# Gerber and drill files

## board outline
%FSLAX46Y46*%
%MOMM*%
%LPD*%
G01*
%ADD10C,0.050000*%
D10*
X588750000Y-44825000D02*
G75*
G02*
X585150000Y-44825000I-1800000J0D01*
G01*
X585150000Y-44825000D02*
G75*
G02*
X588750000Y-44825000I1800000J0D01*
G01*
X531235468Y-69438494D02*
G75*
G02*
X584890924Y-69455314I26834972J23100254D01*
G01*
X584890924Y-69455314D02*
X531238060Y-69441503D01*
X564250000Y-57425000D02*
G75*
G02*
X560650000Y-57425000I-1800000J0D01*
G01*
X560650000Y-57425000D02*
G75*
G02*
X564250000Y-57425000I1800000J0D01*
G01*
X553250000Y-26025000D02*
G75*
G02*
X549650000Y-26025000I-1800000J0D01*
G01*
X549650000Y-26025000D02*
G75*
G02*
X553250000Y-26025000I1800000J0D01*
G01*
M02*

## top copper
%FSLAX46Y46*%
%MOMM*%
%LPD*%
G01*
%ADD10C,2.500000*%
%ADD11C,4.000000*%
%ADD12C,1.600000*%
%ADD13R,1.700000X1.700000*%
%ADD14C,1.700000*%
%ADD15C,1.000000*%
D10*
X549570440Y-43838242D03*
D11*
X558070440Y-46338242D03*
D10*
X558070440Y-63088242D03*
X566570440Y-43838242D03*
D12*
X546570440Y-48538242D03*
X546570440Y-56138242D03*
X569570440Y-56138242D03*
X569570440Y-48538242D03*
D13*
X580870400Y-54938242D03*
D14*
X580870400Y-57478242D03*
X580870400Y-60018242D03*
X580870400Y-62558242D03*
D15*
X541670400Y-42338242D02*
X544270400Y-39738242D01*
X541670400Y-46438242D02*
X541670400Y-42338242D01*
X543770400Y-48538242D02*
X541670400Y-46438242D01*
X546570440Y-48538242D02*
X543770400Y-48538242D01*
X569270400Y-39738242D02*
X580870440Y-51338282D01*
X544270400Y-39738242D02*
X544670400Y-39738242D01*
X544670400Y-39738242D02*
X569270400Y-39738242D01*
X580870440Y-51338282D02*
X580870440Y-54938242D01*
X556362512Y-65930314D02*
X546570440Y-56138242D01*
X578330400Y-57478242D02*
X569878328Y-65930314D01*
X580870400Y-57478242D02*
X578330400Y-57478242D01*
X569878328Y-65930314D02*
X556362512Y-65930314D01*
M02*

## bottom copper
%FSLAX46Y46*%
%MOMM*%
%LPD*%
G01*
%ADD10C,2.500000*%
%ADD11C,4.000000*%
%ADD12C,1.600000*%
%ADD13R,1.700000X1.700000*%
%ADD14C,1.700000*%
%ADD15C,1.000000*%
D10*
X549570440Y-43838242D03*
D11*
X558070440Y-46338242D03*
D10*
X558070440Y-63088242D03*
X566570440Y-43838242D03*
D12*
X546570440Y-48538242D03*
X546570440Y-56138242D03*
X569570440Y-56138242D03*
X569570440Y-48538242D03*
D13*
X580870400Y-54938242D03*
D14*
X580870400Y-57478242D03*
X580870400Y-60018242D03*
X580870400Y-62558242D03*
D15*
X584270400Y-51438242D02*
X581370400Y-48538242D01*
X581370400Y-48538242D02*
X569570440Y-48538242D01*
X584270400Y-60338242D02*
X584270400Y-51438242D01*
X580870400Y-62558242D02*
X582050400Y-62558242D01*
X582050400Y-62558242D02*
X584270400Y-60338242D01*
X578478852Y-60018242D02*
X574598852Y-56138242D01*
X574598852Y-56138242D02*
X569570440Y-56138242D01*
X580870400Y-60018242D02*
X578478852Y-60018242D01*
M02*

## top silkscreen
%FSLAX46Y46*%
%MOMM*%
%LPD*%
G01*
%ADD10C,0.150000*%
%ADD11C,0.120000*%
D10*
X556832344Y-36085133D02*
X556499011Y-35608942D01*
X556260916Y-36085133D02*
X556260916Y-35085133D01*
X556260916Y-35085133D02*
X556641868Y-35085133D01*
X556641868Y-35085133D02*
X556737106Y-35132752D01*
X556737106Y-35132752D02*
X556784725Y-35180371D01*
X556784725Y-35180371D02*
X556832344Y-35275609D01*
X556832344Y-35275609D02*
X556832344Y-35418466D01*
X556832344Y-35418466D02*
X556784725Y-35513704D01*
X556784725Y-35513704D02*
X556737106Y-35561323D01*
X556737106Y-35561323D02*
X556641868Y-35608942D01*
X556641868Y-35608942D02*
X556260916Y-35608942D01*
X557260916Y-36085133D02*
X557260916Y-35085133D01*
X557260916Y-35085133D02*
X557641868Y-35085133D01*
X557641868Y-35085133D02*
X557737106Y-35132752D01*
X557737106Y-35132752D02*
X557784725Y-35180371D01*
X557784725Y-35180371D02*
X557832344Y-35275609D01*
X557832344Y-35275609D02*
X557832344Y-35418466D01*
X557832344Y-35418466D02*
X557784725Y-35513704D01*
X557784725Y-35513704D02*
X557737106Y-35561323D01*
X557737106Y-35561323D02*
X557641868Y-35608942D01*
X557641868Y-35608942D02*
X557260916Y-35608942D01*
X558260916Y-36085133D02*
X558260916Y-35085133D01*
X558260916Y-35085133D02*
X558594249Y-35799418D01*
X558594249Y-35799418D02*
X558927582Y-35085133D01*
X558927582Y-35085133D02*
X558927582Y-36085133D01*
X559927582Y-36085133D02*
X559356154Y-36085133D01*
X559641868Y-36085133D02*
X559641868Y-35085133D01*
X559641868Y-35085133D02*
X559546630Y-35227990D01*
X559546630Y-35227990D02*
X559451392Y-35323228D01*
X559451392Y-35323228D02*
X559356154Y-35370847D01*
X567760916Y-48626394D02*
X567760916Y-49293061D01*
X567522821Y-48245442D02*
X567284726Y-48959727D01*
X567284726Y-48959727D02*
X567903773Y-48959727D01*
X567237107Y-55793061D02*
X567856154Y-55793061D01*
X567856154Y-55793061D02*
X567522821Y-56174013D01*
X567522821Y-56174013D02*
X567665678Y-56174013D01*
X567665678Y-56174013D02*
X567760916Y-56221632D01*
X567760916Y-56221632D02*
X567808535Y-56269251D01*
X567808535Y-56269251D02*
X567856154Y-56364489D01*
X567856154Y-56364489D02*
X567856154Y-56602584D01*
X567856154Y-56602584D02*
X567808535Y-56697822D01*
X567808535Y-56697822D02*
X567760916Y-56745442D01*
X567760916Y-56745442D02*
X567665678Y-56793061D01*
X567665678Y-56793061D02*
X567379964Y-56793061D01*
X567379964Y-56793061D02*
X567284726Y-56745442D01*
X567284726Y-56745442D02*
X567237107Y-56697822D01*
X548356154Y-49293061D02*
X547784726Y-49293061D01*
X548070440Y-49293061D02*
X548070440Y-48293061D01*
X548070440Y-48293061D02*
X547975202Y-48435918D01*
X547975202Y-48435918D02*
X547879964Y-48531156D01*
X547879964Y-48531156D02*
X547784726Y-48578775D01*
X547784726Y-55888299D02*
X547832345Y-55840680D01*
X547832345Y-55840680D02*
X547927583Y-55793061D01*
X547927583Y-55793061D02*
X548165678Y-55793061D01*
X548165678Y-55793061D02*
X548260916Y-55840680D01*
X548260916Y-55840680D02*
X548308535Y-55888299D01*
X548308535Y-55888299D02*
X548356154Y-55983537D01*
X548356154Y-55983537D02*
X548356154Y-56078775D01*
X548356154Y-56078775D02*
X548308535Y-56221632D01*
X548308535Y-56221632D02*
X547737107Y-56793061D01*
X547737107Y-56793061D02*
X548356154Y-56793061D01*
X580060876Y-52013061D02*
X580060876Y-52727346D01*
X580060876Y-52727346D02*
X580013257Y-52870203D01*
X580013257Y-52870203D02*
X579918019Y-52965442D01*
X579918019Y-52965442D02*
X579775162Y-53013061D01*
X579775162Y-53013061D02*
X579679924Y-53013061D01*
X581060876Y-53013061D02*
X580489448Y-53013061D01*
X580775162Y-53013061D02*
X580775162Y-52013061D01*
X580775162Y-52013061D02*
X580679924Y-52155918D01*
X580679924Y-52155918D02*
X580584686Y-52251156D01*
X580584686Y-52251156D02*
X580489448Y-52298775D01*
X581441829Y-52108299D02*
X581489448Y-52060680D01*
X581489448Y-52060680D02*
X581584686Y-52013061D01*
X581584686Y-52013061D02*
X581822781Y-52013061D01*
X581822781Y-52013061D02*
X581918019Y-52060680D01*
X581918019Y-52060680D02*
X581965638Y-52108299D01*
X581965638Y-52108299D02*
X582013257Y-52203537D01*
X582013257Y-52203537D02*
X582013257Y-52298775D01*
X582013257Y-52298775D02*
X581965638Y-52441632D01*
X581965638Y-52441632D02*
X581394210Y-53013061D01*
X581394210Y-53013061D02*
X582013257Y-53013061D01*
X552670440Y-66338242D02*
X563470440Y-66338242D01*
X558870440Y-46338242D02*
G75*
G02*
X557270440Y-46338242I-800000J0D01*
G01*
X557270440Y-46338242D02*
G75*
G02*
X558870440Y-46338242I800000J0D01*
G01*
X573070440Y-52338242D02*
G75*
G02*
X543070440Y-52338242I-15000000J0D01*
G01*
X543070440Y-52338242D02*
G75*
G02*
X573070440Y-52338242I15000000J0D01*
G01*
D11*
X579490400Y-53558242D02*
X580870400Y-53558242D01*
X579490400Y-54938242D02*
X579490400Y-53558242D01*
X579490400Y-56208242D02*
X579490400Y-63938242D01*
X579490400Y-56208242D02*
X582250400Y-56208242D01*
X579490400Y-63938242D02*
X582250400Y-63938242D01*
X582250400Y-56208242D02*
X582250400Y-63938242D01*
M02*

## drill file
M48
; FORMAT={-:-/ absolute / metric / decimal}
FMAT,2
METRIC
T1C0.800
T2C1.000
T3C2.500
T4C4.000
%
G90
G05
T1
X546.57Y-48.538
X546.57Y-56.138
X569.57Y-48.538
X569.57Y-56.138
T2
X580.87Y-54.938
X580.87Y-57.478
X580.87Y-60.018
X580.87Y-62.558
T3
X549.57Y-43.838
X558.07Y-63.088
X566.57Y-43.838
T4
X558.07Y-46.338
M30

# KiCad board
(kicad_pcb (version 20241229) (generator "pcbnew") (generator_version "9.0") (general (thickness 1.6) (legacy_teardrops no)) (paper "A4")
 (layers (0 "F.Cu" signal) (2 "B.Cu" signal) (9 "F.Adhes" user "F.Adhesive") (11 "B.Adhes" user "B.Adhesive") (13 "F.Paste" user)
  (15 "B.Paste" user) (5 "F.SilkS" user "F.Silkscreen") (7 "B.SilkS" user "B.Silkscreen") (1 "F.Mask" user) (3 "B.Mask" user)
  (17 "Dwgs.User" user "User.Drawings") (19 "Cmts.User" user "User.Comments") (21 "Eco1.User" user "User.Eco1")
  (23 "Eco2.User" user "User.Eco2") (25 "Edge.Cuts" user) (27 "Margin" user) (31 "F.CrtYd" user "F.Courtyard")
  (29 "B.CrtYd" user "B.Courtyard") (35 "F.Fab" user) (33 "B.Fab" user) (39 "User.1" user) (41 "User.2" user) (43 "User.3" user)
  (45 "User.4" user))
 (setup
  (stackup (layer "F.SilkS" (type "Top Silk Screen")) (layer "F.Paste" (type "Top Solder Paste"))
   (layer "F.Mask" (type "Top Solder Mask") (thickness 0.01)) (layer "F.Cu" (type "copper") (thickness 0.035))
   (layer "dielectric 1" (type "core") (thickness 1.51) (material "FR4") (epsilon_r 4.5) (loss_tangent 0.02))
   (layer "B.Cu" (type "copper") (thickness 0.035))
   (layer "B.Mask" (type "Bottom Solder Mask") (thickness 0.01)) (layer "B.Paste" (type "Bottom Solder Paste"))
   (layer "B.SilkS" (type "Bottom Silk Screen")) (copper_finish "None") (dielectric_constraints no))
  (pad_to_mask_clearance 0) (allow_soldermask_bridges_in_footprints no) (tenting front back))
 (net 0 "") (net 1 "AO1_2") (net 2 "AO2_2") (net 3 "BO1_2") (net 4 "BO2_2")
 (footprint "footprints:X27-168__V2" (layer "F.Cu") (at 558.07044 52.338242)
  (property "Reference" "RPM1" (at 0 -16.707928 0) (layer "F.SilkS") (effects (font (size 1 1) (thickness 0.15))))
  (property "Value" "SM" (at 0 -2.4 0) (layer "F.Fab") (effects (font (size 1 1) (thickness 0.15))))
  (fp_line (start -5.4 14) (end 5.4 14) (stroke (width 0.15) (type solid)) (layer "F.SilkS"))
  (fp_circle (center 0 -6) (end 0.8 -6) (stroke (width 0.15) (type solid)) (fill no) (layer "F.SilkS"))
  (fp_circle (center 0 0) (end 15 0) (stroke (width 0.15) (type solid)) (fill no) (layer "F.SilkS"))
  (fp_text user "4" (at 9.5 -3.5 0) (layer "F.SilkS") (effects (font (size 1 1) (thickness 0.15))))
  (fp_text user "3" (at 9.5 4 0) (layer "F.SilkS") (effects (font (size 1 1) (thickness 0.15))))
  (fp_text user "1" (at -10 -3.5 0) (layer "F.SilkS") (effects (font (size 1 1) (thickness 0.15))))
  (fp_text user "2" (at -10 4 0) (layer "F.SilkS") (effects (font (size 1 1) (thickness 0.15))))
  (pad "" thru_hole circle (at -8.5 -8.5) (size 2.5 2.5) (drill 2.5) (layers "*.Cu" "*.Mask") (remove_unused_layers no))
  (pad "" thru_hole circle (at 0 -6) (size 4 4) (drill 4) (layers "*.Cu" "*.Mask") (remove_unused_layers no))
  (pad "" thru_hole circle (at 0 10.75) (size 2.5 2.5) (drill 2.5) (layers "*.Cu" "*.Mask") (remove_unused_layers no))
  (pad "" thru_hole circle (at 8.5 -8.5) (size 2.5 2.5) (drill 2.5) (layers "*.Cu" "*.Mask") (remove_unused_layers no))
  (pad "1" thru_hole circle (at -11.5 -3.8) (size 1.6 1.6) (drill 0.8) (layers "*.Cu" "*.Mask") (remove_unused_layers no) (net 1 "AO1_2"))
  (pad "2" thru_hole circle (at -11.5 3.8) (size 1.6 1.6) (drill 0.8) (layers "*.Cu" "*.Mask") (remove_unused_layers no) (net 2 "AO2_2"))
  (pad "3" thru_hole circle (at 11.5 3.8) (size 1.6 1.6) (drill 0.8) (layers "*.Cu" "*.Mask") (remove_unused_layers no) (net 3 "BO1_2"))
  (pad "4" thru_hole circle (at 11.5 -3.8) (size 1.6 1.6) (drill 0.8) (layers "*.Cu" "*.Mask") (remove_unused_layers no) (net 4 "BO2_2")))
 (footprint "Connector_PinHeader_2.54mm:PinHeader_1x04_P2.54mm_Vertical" (layer "F.Cu") (at 580.8704 54.938242)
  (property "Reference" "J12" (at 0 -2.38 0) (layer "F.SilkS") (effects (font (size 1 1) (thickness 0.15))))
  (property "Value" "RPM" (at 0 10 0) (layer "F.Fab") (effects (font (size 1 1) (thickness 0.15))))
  (fp_line (start -1.38 -1.38) (end 0 -1.38) (stroke (width 0.12) (type solid)) (layer "F.SilkS"))
  (fp_line (start -1.38 0) (end -1.38 -1.38) (stroke (width 0.12) (type solid)) (layer "F.SilkS"))
  (fp_line (start -1.38 1.27) (end -1.38 9) (stroke (width 0.12) (type solid)) (layer "F.SilkS"))
  (fp_line (start -1.38 1.27) (end 1.38 1.27) (stroke (width 0.12) (type solid)) (layer "F.SilkS"))
  (fp_line (start -1.38 9) (end 1.38 9) (stroke (width 0.12) (type solid)) (layer "F.SilkS"))
  (fp_line (start 1.38 1.27) (end 1.38 9) (stroke (width 0.12) (type solid)) (layer "F.SilkS"))
  (pad "1" thru_hole rect (at 0 0) (size 1.7 1.7) (drill 1) (layers "*.Cu" "*.Mask") (remove_unused_layers no) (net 1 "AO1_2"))
  (pad "2" thru_hole circle (at 0 2.54) (size 1.7 1.7) (drill 1) (layers "*.Cu" "*.Mask") (remove_unused_layers no) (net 2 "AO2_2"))
  (pad "3" thru_hole circle (at 0 5.08) (size 1.7 1.7) (drill 1) (layers "*.Cu" "*.Mask") (remove_unused_layers no) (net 3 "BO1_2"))
  (pad "4" thru_hole circle (at 0 7.62) (size 1.7 1.7) (drill 1) (layers "*.Cu" "*.Mask") (remove_unused_layers no) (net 4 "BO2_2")))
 (gr_circle (center 586.95 44.825) (end 585.15 44.825) (stroke (width 0.05) (type default)) (fill no) (layer "Edge.Cuts"))
 (gr_arc (start 531.235468 69.438494) (mid 558.08154 10.93009) (end 584.890924 69.455314) (stroke (width 0.05) (type default))
  (layer "Edge.Cuts"))
 (gr_line (start 584.890924 69.455314) (end 531.23806 69.441503) (stroke (width 0.05) (type default)) (layer "Edge.Cuts"))
 (gr_circle (center 562.45 57.425) (end 560.65 57.425) (stroke (width 0.05) (type default)) (fill no) (layer "Edge.Cuts"))
 (gr_circle (center 551.45 26.025) (end 549.65 26.025) (stroke (width 0.05) (type default)) (fill no) (layer "Edge.Cuts"))
 (segment (start 541.6704 42.338242) (end 544.2704 39.738242) (width 1) (layer "F.Cu") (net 1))
 (segment (start 541.6704 46.438242) (end 541.6704 42.338242) (width 1) (layer "F.Cu") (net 1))
 (segment (start 543.7704 48.538242) (end 541.6704 46.438242) (width 1) (layer "F.Cu") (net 1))
 (segment (start 546.57044 48.538242) (end 543.7704 48.538242) (width 1) (layer "F.Cu") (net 1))
 (segment (start 569.2704 39.738242) (end 580.87044 51.338282) (width 1) (layer "F.Cu") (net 1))
 (segment (start 544.2704 39.738242) (end 544.6704 39.738242) (width 1) (layer "F.Cu") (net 1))
 (segment (start 544.6704 39.738242) (end 569.2704 39.738242) (width 1) (layer "F.Cu") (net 1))
 (segment (start 580.87044 51.338282) (end 580.87044 54.938242) (width 1) (layer "F.Cu") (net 1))
 (segment (start 556.362512 65.930314) (end 546.57044 56.138242) (width 1) (layer "F.Cu") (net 2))
 (segment (start 578.3304 57.478242) (end 569.878328 65.930314) (width 1) (layer "F.Cu") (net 2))
 (segment (start 580.8704 57.478242) (end 578.3304 57.478242) (width 1) (layer "F.Cu") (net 2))
 (segment (start 569.878328 65.930314) (end 556.362512 65.930314) (width 1) (layer "F.Cu") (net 2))
 (segment (start 584.2704 51.438242) (end 581.3704 48.538242) (width 1) (layer "B.Cu") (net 4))
 (segment (start 581.3704 48.538242) (end 569.57044 48.538242) (width 1) (layer "B.Cu") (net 4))
 (segment (start 584.2704 60.338242) (end 584.2704 51.438242) (width 1) (layer "B.Cu") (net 4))
 (segment (start 580.8704 62.558242) (end 582.0504 62.558242) (width 1) (layer "B.Cu") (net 4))
 (segment (start 582.0504 62.558242) (end 584.2704 60.338242) (width 1) (layer "B.Cu") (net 4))
 (segment (start 578.478852 60.018242) (end 574.598852 56.138242) (width 1) (layer "B.Cu") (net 3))
 (segment (start 574.598852 56.138242) (end 569.57044 56.138242) (width 1) (layer "B.Cu") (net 3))
 (segment (start 580.8704 60.018242) (end 578.478852 60.018242) (width 1) (layer "B.Cu") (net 3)))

